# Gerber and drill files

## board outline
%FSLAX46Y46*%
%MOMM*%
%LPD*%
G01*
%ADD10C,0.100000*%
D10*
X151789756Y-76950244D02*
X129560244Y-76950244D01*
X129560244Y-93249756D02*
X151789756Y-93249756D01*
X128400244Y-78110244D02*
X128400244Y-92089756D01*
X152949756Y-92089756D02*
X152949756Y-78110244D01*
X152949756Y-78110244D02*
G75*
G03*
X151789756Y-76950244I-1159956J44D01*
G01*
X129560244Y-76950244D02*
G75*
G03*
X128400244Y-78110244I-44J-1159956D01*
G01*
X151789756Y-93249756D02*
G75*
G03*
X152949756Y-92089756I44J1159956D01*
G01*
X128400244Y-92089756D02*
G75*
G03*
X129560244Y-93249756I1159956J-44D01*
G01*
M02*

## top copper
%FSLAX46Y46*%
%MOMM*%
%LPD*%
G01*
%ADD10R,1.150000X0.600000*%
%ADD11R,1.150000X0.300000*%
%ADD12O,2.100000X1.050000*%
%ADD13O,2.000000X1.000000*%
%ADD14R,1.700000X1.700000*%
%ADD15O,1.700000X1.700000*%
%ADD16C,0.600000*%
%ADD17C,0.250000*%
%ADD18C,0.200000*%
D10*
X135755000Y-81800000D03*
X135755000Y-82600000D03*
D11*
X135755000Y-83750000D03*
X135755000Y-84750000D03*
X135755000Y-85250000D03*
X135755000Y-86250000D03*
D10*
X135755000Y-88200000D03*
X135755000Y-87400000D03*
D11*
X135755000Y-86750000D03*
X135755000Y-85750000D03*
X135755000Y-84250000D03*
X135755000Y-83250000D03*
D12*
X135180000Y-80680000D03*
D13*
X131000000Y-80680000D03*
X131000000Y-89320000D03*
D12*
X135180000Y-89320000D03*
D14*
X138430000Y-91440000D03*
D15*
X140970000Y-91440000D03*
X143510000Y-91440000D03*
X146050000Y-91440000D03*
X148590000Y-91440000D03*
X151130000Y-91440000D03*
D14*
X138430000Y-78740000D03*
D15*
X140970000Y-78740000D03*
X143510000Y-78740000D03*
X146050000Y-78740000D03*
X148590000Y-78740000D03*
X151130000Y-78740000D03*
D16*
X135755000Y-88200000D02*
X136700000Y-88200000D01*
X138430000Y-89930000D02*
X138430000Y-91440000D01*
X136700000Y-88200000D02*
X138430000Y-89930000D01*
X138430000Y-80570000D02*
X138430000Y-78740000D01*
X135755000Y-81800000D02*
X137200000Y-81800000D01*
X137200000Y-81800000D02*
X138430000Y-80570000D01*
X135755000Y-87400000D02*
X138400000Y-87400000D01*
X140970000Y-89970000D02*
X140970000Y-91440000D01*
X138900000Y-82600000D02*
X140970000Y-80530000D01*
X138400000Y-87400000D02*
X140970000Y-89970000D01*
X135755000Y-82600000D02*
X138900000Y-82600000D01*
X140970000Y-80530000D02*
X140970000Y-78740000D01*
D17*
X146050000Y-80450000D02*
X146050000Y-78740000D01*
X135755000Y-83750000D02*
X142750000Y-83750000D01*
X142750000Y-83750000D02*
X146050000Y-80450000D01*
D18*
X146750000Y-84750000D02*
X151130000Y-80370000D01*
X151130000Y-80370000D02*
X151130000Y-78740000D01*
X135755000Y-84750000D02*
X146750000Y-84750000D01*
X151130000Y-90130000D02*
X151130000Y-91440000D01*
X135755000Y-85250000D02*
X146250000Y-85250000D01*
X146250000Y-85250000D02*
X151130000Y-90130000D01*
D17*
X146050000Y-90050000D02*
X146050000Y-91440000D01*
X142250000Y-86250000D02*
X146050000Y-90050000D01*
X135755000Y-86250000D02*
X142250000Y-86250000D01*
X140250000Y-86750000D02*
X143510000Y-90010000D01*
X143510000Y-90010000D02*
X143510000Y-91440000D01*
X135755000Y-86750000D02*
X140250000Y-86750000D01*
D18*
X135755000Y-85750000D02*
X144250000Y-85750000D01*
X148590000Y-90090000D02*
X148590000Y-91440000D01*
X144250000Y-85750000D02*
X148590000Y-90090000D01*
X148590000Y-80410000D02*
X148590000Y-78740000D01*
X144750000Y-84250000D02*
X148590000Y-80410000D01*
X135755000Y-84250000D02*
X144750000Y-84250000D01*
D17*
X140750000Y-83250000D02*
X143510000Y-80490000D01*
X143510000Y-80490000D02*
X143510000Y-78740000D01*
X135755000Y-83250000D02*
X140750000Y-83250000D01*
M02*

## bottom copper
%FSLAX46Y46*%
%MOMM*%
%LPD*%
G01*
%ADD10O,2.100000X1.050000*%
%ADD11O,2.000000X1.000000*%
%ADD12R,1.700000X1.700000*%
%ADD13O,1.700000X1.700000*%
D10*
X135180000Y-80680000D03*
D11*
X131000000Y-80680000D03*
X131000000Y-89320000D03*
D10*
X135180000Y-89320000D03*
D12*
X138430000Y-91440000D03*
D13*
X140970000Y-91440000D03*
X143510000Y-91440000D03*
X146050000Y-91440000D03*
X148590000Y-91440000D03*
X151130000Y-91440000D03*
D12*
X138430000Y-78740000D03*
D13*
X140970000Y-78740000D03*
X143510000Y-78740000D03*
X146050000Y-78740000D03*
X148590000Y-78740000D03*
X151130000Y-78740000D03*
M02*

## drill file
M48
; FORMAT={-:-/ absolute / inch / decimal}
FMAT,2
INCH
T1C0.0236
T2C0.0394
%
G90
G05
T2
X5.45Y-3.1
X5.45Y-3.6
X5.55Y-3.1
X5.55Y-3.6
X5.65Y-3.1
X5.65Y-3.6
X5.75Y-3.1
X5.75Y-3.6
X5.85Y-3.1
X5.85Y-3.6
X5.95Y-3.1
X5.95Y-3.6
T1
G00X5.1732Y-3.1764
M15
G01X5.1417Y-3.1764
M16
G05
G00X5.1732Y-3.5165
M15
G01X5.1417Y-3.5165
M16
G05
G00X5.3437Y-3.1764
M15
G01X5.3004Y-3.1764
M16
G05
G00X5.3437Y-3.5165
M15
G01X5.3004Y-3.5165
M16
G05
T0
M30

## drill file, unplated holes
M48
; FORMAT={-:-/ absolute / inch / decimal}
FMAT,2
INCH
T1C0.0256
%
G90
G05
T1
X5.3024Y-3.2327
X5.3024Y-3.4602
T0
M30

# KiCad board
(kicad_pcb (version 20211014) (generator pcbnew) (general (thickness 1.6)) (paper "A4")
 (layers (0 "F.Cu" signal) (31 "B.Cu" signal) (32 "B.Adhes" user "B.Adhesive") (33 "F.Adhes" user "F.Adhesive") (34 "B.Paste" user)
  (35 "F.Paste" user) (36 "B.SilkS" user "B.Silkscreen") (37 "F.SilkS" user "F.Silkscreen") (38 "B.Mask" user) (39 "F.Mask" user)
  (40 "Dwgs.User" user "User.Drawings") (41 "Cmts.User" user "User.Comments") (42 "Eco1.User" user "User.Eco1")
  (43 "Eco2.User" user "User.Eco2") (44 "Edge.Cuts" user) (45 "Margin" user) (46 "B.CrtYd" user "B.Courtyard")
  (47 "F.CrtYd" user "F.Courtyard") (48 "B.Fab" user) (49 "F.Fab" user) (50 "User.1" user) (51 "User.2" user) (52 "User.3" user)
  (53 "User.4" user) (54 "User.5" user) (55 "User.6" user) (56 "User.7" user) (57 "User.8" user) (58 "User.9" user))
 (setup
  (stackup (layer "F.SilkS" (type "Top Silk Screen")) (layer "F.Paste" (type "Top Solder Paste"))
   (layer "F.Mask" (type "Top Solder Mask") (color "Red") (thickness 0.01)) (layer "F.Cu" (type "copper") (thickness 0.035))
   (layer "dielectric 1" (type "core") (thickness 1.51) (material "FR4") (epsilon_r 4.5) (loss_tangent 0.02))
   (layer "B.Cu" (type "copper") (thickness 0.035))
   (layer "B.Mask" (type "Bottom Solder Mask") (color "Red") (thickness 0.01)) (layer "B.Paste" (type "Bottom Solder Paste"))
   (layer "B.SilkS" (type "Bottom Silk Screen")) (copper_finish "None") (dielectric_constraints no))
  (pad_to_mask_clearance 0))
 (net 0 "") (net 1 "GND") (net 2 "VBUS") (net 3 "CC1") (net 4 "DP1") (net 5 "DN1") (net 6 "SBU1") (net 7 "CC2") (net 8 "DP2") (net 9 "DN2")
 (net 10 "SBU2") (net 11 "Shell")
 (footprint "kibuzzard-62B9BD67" (layer "F.Cu") (at 148.59 82.042 90)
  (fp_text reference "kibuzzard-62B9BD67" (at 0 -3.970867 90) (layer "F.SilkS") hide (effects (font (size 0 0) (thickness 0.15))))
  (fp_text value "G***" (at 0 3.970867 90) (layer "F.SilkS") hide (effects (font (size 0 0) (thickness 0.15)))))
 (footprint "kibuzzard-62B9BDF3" (layer "F.Cu") (at 140.97 88.138 90)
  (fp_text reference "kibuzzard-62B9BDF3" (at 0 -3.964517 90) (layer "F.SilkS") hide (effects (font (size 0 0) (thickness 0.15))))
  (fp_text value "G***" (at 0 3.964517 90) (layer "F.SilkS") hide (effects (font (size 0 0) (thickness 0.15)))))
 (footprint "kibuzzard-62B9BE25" (layer "F.Cu") (at 148.59 88.138 90)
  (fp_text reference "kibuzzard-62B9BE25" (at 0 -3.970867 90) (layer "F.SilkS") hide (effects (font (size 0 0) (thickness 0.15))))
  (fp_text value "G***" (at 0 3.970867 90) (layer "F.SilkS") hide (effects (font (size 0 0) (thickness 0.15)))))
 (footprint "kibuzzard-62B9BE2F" (layer "F.Cu") (at 151.13 88.138 90)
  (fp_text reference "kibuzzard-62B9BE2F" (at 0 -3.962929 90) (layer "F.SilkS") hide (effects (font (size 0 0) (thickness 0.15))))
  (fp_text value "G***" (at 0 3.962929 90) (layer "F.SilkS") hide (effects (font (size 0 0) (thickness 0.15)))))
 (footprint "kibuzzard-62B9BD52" (layer "F.Cu") (at 146.05 81.788 90)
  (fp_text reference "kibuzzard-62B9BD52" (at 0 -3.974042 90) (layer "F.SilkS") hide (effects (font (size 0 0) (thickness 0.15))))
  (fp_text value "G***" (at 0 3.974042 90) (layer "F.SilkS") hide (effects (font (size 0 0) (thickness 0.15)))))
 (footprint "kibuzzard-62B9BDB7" (layer "F.Cu") (at 140.97 82.042 90)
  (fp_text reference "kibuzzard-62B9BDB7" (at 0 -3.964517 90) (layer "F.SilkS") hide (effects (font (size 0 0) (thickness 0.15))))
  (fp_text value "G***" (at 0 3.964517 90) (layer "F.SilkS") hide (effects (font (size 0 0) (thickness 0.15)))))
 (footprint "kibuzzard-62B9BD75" (layer "F.Cu") (at 151.13 81.788 90)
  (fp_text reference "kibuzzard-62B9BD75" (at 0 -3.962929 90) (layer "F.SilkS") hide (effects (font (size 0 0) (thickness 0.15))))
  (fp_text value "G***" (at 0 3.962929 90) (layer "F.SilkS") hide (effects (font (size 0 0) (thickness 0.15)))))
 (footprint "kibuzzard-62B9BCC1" (layer "F.Cu") (at 138.43 88.138 90)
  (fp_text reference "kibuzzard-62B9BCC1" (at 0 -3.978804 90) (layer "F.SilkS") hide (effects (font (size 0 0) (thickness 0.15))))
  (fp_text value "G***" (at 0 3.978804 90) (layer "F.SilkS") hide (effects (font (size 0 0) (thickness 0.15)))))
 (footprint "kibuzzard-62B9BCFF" (layer "F.Cu") (at 138.43 82.042 90)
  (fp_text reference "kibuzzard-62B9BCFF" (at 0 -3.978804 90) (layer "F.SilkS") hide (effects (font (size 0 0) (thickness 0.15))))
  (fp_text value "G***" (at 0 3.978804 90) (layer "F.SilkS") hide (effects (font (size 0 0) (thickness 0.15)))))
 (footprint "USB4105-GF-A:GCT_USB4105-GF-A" (layer "F.Cu") (at 131 85 -90)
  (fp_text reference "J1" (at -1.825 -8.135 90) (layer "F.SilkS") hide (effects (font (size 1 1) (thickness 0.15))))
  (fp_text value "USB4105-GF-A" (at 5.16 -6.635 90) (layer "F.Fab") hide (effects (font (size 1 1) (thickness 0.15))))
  (pad "" np_thru_hole circle (at 2.89 -3.68 270) (size 0.65 0.65) (drill 0.65) (layers *.Cu *.Mask))
  (pad "" np_thru_hole circle (at -2.89 -3.68 270) (size 0.65 0.65) (drill 0.65) (layers *.Cu *.Mask))
  (pad "A1_B12" smd rect (at -3.2 -4.755 270) (size 0.6 1.15) (layers "F.Cu" "F.Paste" "F.Mask") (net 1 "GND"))
  (pad "A4_B9" smd rect (at -2.4 -4.755 270) (size 0.6 1.15) (layers "F.Cu" "F.Paste" "F.Mask") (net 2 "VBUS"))
  (pad "A5" smd rect (at -1.25 -4.755 270) (size 0.3 1.15) (layers "F.Cu" "F.Paste" "F.Mask") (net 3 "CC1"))
  (pad "A6" smd rect (at -0.25 -4.755 270) (size 0.3 1.15) (layers "F.Cu" "F.Paste" "F.Mask") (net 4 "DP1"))
  (pad "A7" smd rect (at 0.25 -4.755 270) (size 0.3 1.15) (layers "F.Cu" "F.Paste" "F.Mask") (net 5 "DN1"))
  (pad "A8" smd rect (at 1.25 -4.755 270) (size 0.3 1.15) (layers "F.Cu" "F.Paste" "F.Mask") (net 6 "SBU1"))
  (pad "B1_A12" smd rect (at 3.2 -4.755 270) (size 0.6 1.15) (layers "F.Cu" "F.Paste" "F.Mask") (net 1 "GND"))
  (pad "B4_A9" smd rect (at 2.4 -4.755 270) (size 0.6 1.15) (layers "F.Cu" "F.Paste" "F.Mask") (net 2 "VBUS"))
  (pad "B5" smd rect (at 1.75 -4.755 270) (size 0.3 1.15) (layers "F.Cu" "F.Paste" "F.Mask") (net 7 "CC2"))
  (pad "B6" smd rect (at 0.75 -4.755 270) (size 0.3 1.15) (layers "F.Cu" "F.Paste" "F.Mask") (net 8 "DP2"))
  (pad "B7" smd rect (at -0.75 -4.755 270) (size 0.3 1.15) (layers "F.Cu" "F.Paste" "F.Mask") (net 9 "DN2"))
  (pad "B8" smd rect (at -1.75 -4.755 270) (size 0.3 1.15) (layers "F.Cu" "F.Paste" "F.Mask") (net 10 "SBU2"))
  (pad "S1" thru_hole oval (at -4.32 -4.18 270) (size 1.05 2.1) (drill oval 0.6 1.7) (layers *.Cu *.Mask) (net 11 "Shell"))
  (pad "S2" thru_hole oval (at -4.32 0 270) (size 1 2) (drill oval 0.6 1.4) (layers *.Cu *.Mask) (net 11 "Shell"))
  (pad "S3" thru_hole oval (at 4.32 0 270) (size 1 2) (drill oval 0.6 1.4) (layers *.Cu *.Mask) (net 11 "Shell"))
  (pad "S4" thru_hole oval (at 4.32 -4.18 270) (size 1.05 2.1) (drill oval 0.6 1.7) (layers *.Cu *.Mask) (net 11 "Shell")))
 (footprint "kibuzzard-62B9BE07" (layer "F.Cu") (at 143.51 88.138 90)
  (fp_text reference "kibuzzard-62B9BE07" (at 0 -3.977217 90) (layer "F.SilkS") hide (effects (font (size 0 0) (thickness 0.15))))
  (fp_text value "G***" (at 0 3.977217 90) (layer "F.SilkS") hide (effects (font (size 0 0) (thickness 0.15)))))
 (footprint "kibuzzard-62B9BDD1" (layer "F.Cu") (at 143.51 81.788 90)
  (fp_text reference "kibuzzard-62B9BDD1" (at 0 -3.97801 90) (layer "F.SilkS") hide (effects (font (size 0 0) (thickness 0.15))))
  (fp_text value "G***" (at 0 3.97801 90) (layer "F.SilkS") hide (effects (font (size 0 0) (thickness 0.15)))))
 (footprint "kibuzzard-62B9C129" (layer "F.Cu") (at 146.07 88.39 90)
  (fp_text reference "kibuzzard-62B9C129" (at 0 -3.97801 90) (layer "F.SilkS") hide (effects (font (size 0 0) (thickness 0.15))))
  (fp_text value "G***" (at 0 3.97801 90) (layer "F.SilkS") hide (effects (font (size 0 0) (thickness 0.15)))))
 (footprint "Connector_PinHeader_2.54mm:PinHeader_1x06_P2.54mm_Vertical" (layer "B.Cu") (at 138.43 91.44 -90)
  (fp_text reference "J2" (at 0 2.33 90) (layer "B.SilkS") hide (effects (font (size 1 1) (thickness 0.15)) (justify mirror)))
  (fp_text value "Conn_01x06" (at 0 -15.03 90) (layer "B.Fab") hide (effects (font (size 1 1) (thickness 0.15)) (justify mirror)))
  (pad "1" thru_hole rect (at 0 0 270) (size 1.7 1.7) (drill 1) (layers *.Cu *.Mask) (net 1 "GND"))
  (pad "2" thru_hole oval (at 0 -2.54 270) (size 1.7 1.7) (drill 1) (layers *.Cu *.Mask) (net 2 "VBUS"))
  (pad "3" thru_hole oval (at 0 -5.08 270) (size 1.7 1.7) (drill 1) (layers *.Cu *.Mask) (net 7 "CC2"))
  (pad "4" thru_hole oval (at 0 -7.62 270) (size 1.7 1.7) (drill 1) (layers *.Cu *.Mask) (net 6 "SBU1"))
  (pad "5" thru_hole oval (at 0 -10.16 270) (size 1.7 1.7) (drill 1) (layers *.Cu *.Mask) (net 8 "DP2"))
  (pad "6" thru_hole oval (at 0 -12.7 270) (size 1.7 1.7) (drill 1) (layers *.Cu *.Mask) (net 5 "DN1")))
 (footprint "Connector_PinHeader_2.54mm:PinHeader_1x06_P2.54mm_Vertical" (layer "B.Cu") (at 138.43 78.74 -90)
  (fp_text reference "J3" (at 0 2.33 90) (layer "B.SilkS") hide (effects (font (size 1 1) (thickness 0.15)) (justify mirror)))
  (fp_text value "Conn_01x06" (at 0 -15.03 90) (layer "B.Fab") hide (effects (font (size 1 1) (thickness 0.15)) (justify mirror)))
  (pad "1" thru_hole rect (at 0 0 270) (size 1.7 1.7) (drill 1) (layers *.Cu *.Mask) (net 1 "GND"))
  (pad "2" thru_hole oval (at 0 -2.54 270) (size 1.7 1.7) (drill 1) (layers *.Cu *.Mask) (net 2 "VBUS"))
  (pad "3" thru_hole oval (at 0 -5.08 270) (size 1.7 1.7) (drill 1) (layers *.Cu *.Mask) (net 10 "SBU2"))
  (pad "4" thru_hole oval (at 0 -7.62 270) (size 1.7 1.7) (drill 1) (layers *.Cu *.Mask) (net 3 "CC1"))
  (pad "5" thru_hole oval (at 0 -10.16 270) (size 1.7 1.7) (drill 1) (layers *.Cu *.Mask) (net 9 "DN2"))
  (pad "6" thru_hole oval (at 0 -12.7 270) (size 1.7 1.7) (drill 1) (layers *.Cu *.Mask) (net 4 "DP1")))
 (gr_line (start 151.789756 76.950244) (end 129.560244 76.950244) (layer "Edge.Cuts") (width 0.1))
 (gr_line (start 129.560244 93.249756) (end 151.789756 93.249756) (layer "Edge.Cuts") (width 0.1))
 (gr_line (start 128.400244 78.110244) (end 128.400244 92.089756) (layer "Edge.Cuts") (width 0.1))
 (gr_line (start 152.949756 92.089756) (end 152.949756 78.110244) (layer "Edge.Cuts") (width 0.1))
 (gr_arc (start 151.789756 76.950244) (mid 152.61 77.29) (end 152.949756 78.110244) (layer "Edge.Cuts") (width 0.1))
 (gr_arc (start 128.400244 78.110244) (mid 128.74 77.29) (end 129.560244 76.950244) (layer "Edge.Cuts") (width 0.1))
 (gr_arc (start 152.949756 92.089756) (mid 152.61 92.91) (end 151.789756 93.249756) (layer "Edge.Cuts") (width 0.1))
 (gr_arc (start 129.560244 93.249756) (mid 128.74 92.91) (end 128.400244 92.089756) (layer "Edge.Cuts") (width 0.1))
 (segment (start 135.755 88.2) (end 136.7 88.2) (width 0.6) (layer "F.Cu") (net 1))
 (segment (start 138.43 89.93) (end 138.43 91.44) (width 0.6) (layer "F.Cu") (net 1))
 (segment (start 136.7 88.2) (end 138.43 89.93) (width 0.6) (layer "F.Cu") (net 1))
 (segment (start 138.43 80.57) (end 138.43 78.74) (width 0.6) (layer "F.Cu") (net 1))
 (segment (start 135.755 81.8) (end 137.2 81.8) (width 0.6) (layer "F.Cu") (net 1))
 (segment (start 137.2 81.8) (end 138.43 80.57) (width 0.6) (layer "F.Cu") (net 1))
 (segment (start 135.755 87.4) (end 138.4 87.4) (width 0.6) (layer "F.Cu") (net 2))
 (segment (start 140.97 89.97) (end 140.97 91.44) (width 0.6) (layer "F.Cu") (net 2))
 (segment (start 138.9 82.6) (end 140.97 80.53) (width 0.6) (layer "F.Cu") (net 2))
 (segment (start 138.4 87.4) (end 140.97 89.97) (width 0.6) (layer "F.Cu") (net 2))
 (segment (start 135.755 82.6) (end 138.9 82.6) (width 0.6) (layer "F.Cu") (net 2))
 (segment (start 140.97 80.53) (end 140.97 78.74) (width 0.6) (layer "F.Cu") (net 2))
 (segment (start 146.05 80.45) (end 146.05 78.74) (width 0.25) (layer "F.Cu") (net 3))
 (segment (start 135.755 83.75) (end 142.75 83.75) (width 0.25) (layer "F.Cu") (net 3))
 (segment (start 142.75 83.75) (end 146.05 80.45) (width 0.25) (layer "F.Cu") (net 3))
 (segment (start 146.75 84.75) (end 151.13 80.37) (width 0.2) (layer "F.Cu") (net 4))
 (segment (start 151.13 80.37) (end 151.13 78.74) (width 0.2) (layer "F.Cu") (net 4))
 (segment (start 135.755 84.75) (end 146.75 84.75) (width 0.2) (layer "F.Cu") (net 4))
 (segment (start 151.13 90.13) (end 151.13 91.44) (width 0.2) (layer "F.Cu") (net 5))
 (segment (start 135.755 85.25) (end 146.25 85.25) (width 0.2) (layer "F.Cu") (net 5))
 (segment (start 146.25 85.25) (end 151.13 90.13) (width 0.2) (layer "F.Cu") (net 5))
 (segment (start 146.05 90.05) (end 146.05 91.44) (width 0.25) (layer "F.Cu") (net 6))
 (segment (start 142.25 86.25) (end 146.05 90.05) (width 0.25) (layer "F.Cu") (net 6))
 (segment (start 135.755 86.25) (end 142.25 86.25) (width 0.25) (layer "F.Cu") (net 6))
 (segment (start 140.25 86.75) (end 143.51 90.01) (width 0.25) (layer "F.Cu") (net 7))
 (segment (start 143.51 90.01) (end 143.51 91.44) (width 0.25) (layer "F.Cu") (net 7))
 (segment (start 135.755 86.75) (end 140.25 86.75) (width 0.25) (layer "F.Cu") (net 7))
 (segment (start 135.755 85.75) (end 144.25 85.75) (width 0.2) (layer "F.Cu") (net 8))
 (segment (start 148.59 90.09) (end 148.59 91.44) (width 0.2) (layer "F.Cu") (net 8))
 (segment (start 144.25 85.75) (end 148.59 90.09) (width 0.2) (layer "F.Cu") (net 8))
 (segment (start 148.59 80.41) (end 148.59 78.74) (width 0.2) (layer "F.Cu") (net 9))
 (segment (start 144.75 84.25) (end 148.59 80.41) (width 0.2) (layer "F.Cu") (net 9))
 (segment (start 135.755 84.25) (end 144.75 84.25) (width 0.2) (layer "F.Cu") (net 9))
 (segment (start 140.75 83.25) (end 143.51 80.49) (width 0.25) (layer "F.Cu") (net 10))
 (segment (start 143.51 80.49) (end 143.51 78.74) (width 0.25) (layer "F.Cu") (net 10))
 (segment (start 135.755 83.25) (end 140.75 83.25) (width 0.25) (layer "F.Cu") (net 10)))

